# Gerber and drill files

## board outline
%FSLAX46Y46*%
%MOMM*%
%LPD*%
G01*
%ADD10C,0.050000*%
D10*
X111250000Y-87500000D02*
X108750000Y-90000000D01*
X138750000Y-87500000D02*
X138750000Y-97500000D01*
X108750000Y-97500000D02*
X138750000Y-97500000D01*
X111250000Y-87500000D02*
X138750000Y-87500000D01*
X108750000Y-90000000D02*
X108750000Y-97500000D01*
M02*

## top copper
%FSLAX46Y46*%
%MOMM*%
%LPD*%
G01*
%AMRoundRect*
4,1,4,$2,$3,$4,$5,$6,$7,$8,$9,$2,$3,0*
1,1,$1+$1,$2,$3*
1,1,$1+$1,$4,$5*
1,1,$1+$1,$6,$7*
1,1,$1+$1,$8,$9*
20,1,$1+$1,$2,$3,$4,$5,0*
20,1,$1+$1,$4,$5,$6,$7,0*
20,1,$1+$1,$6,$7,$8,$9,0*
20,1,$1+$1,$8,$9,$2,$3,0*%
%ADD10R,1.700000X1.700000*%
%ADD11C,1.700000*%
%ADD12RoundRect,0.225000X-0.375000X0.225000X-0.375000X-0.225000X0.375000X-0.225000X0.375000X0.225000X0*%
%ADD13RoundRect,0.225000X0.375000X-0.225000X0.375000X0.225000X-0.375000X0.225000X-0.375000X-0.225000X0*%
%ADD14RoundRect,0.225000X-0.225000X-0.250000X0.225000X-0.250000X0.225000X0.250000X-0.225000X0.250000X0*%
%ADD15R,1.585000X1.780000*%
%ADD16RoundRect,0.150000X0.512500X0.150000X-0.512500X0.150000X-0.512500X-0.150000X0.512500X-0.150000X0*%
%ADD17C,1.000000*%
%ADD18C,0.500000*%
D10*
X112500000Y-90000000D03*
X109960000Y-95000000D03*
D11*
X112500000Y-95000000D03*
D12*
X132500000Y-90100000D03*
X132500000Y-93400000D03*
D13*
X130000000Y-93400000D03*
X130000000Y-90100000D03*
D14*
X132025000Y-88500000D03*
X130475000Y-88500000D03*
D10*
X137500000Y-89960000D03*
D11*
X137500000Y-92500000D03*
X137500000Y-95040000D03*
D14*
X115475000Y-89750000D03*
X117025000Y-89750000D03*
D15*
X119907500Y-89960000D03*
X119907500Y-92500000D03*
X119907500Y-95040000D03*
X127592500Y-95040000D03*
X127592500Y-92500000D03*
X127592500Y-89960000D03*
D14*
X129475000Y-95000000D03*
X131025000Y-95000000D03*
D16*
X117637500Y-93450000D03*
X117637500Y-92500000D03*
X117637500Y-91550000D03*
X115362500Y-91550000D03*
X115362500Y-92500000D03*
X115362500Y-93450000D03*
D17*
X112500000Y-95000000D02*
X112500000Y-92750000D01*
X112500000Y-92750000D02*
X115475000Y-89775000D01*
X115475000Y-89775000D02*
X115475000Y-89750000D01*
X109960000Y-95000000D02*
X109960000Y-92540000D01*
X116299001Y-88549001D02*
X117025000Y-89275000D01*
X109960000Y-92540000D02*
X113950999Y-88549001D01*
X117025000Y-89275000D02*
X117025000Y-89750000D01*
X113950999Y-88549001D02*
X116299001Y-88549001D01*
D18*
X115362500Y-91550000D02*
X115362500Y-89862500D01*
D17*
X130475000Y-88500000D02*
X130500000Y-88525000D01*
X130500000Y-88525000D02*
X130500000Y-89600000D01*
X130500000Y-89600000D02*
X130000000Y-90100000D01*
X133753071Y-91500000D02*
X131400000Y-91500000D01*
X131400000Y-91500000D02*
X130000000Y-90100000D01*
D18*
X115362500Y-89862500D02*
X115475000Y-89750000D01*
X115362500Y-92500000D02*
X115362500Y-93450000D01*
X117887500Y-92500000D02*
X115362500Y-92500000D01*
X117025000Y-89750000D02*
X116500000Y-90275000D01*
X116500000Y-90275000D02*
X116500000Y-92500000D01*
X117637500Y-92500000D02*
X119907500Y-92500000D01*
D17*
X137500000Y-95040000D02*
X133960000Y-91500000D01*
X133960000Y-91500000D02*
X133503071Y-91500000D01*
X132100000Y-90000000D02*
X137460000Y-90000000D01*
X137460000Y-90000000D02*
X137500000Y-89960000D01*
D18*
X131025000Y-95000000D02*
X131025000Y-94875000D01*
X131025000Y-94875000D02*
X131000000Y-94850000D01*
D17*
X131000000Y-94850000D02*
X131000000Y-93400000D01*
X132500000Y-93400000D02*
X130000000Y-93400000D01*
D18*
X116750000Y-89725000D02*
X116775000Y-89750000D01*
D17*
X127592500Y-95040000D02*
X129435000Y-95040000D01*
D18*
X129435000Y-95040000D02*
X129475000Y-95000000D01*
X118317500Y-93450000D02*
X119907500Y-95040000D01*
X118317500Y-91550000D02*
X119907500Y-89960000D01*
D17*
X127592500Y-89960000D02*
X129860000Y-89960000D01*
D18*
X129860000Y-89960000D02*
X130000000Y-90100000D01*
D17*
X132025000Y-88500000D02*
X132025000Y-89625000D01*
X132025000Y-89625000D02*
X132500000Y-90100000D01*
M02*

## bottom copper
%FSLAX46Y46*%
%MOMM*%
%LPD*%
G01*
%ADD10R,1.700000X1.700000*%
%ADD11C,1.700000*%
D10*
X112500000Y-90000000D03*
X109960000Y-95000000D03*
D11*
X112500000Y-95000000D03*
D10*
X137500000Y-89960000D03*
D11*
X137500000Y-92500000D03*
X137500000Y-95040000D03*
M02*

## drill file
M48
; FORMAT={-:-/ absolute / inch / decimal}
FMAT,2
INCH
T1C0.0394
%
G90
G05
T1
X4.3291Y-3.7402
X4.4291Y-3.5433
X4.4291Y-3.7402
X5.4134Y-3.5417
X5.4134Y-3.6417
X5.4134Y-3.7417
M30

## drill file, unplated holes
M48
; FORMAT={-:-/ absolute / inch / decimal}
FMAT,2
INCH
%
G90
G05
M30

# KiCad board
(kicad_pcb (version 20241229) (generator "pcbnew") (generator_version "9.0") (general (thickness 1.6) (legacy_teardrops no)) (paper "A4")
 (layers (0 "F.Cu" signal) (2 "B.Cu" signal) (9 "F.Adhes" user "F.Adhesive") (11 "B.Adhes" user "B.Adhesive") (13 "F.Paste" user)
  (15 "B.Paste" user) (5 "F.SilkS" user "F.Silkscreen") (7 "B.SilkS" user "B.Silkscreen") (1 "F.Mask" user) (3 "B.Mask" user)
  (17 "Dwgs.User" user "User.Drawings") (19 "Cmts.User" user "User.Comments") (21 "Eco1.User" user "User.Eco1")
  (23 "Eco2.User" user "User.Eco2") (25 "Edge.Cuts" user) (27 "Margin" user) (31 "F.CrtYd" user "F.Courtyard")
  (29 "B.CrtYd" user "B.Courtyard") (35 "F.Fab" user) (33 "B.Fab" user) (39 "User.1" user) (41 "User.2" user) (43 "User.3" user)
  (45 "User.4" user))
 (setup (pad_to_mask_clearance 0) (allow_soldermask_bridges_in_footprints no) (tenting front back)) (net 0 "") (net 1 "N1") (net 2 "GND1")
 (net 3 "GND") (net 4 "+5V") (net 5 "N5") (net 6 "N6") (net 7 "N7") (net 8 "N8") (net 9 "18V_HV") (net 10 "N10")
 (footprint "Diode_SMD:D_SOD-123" (layer "F.Cu") (at 130 91.75 90)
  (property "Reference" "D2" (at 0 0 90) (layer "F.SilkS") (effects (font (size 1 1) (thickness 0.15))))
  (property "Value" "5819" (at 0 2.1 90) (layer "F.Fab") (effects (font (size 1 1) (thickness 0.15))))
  (pad "1" smd roundrect (at -1.65 0 90) (size 0.9 1.2) (layers "F.Cu" "F.Mask" "F.Paste") (roundrect_rratio 0.25) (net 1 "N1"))
  (pad "2" smd roundrect (at 1.65 0 90) (size 0.9 1.2) (layers "F.Cu" "F.Mask" "F.Paste") (roundrect_rratio 0.25) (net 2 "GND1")))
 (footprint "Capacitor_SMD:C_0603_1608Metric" (layer "F.Cu") (at 116.25 89.75)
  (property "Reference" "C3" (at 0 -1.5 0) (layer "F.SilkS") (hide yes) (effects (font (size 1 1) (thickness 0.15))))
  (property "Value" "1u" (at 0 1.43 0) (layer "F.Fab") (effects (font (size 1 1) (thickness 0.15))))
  (pad "1" smd roundrect (at -0.775 0) (size 0.9 0.95) (layers "F.Cu" "F.Mask" "F.Paste") (roundrect_rratio 0.25) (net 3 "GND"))
  (pad "2" smd roundrect (at 0.775 0) (size 0.9 0.95) (layers "F.Cu" "F.Mask" "F.Paste") (roundrect_rratio 0.25) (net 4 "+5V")))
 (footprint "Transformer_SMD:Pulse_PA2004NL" (layer "F.Cu") (at 123.75 92.5)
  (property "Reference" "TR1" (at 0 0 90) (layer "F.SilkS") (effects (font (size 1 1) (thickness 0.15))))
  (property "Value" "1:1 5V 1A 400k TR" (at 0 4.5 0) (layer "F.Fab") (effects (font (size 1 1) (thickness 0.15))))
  (pad "1" smd rect (at -3.8425 -2.54) (size 1.585 1.78) (layers "F.Cu" "F.Mask" "F.Paste") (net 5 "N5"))
  (pad "2" smd rect (at -3.8425 0) (size 1.585 1.78) (layers "F.Cu" "F.Mask" "F.Paste") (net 4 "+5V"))
  (pad "3" smd rect (at -3.8425 2.54) (size 1.585 1.78) (layers "F.Cu" "F.Mask" "F.Paste") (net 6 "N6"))
  (pad "4" smd rect (at 3.8425 2.54) (size 1.585 1.78) (layers "F.Cu" "F.Mask" "F.Paste") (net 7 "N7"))
  (pad "5" smd rect (at 3.8425 0) (size 1.585 1.78) (layers "F.Cu" "F.Mask" "F.Paste") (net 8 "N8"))
  (pad "6" smd rect (at 3.8425 -2.54) (size 1.585 1.78) (layers "F.Cu" "F.Mask" "F.Paste") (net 2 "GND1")))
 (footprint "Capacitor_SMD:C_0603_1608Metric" (layer "F.Cu") (at 130.25 95)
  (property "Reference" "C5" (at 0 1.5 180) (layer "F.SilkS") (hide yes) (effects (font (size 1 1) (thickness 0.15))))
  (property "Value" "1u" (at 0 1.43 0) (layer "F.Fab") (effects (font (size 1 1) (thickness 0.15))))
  (pad "1" smd roundrect (at -0.775 0) (size 0.9 0.95) (layers "F.Cu" "F.Mask" "F.Paste") (roundrect_rratio 0.25) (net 7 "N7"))
  (pad "2" smd roundrect (at 0.775 0) (size 0.9 0.95) (layers "F.Cu" "F.Mask" "F.Paste") (roundrect_rratio 0.25) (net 1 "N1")))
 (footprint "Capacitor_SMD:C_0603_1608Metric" (layer "F.Cu") (at 131.25 88.5)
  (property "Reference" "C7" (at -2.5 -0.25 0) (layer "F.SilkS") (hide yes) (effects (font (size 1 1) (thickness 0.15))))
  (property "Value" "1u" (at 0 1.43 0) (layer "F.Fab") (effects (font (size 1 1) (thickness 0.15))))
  (pad "1" smd roundrect (at -0.775 0) (size 0.9 0.95) (layers "F.Cu" "F.Mask" "F.Paste") (roundrect_rratio 0.25) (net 2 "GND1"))
  (pad "2" smd roundrect (at 0.775 0) (size 0.9 0.95) (layers "F.Cu" "F.Mask" "F.Paste") (roundrect_rratio 0.25) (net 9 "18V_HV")))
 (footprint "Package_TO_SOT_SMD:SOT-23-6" (layer "F.Cu") (at 116.5 92.5 180)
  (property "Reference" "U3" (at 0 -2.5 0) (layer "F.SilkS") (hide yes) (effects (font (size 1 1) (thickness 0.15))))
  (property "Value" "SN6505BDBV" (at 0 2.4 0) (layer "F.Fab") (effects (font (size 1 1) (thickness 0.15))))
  (pad "1" smd roundrect (at -1.1375 -0.95 180) (size 1.325 0.6) (layers "F.Cu" "F.Mask" "F.Paste") (roundrect_rratio 0.25) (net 6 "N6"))
  (pad "2" smd roundrect (at -1.1375 0 180) (size 1.325 0.6) (layers "F.Cu" "F.Mask" "F.Paste") (roundrect_rratio 0.25) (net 4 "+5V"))
  (pad "3" smd roundrect (at -1.1375 0.95 180) (size 1.325 0.6) (layers "F.Cu" "F.Mask" "F.Paste") (roundrect_rratio 0.25) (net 5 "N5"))
  (pad "4" smd roundrect (at 1.1375 0.95 180) (size 1.325 0.6) (layers "F.Cu" "F.Mask" "F.Paste") (roundrect_rratio 0.25) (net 3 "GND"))
  (pad "5" smd roundrect (at 1.1375 0 180) (size 1.325 0.6) (layers "F.Cu" "F.Mask" "F.Paste") (roundrect_rratio 0.25) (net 4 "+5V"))
  (pad "6" smd roundrect (at 1.1375 -0.95 180) (size 1.325 0.6) (layers "F.Cu" "F.Mask" "F.Paste") (roundrect_rratio 0.25) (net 4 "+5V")))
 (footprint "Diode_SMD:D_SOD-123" (layer "F.Cu") (at 132.5 91.75 -90)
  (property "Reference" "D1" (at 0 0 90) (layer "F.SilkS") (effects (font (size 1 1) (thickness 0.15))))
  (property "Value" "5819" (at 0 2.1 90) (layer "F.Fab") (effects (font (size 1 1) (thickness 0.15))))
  (pad "1" smd roundrect (at -1.65 0 270) (size 0.9 1.2) (layers "F.Cu" "F.Mask" "F.Paste") (roundrect_rratio 0.25) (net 9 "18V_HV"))
  (pad "2" smd roundrect (at 1.65 0 270) (size 0.9 1.2) (layers "F.Cu" "F.Mask" "F.Paste") (roundrect_rratio 0.25) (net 1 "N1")))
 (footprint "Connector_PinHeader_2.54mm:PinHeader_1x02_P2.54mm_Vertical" (layer "B.Cu") (at 109.96 95 -90)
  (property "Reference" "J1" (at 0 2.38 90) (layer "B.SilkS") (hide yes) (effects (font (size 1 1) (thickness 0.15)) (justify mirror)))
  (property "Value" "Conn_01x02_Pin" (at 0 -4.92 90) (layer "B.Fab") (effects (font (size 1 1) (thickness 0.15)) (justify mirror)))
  (pad "1" thru_hole rect (at 0 0 270) (size 1.7 1.7) (drill 1) (layers "*.Cu" "*.Mask") (remove_unused_layers no) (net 4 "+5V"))
  (pad "2" thru_hole circle (at 0 -2.54 270) (size 1.7 1.7) (drill 1) (layers "*.Cu" "*.Mask") (remove_unused_layers no) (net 3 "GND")))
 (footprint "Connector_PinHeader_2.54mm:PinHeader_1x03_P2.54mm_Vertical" (layer "B.Cu") (at 137.5 89.96 180)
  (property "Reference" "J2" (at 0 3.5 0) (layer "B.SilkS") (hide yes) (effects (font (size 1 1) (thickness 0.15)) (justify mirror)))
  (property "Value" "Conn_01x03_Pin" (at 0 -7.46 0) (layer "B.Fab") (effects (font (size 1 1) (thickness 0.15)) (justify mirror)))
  (pad "1" thru_hole rect (at 0 0 180) (size 1.7 1.7) (drill 1) (layers "*.Cu" "*.Mask") (remove_unused_layers no) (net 9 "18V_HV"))
  (pad "2" thru_hole circle (at 0 -2.54 180) (size 1.7 1.7) (drill 1) (layers "*.Cu" "*.Mask") (remove_unused_layers no) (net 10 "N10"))
  (pad "3" thru_hole circle (at 0 -5.08 180) (size 1.7 1.7) (drill 1) (layers "*.Cu" "*.Mask") (remove_unused_layers no) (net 2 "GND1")))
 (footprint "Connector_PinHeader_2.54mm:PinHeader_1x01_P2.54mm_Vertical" (layer "B.Cu") (at 112.5 90)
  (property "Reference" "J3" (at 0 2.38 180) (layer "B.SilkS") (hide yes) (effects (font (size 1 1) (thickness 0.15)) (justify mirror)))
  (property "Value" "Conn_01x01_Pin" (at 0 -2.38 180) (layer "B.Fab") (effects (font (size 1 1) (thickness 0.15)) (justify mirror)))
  (pad "1" thru_hole rect (at 0 0) (size 1.7 1.7) (drill 1) (layers "*.Cu" "*.Mask") (remove_unused_layers no) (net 4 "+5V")))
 (gr_line (start 111.25 87.5) (end 138.75 87.5) (stroke (width 0.05) (type default)) (layer "Edge.Cuts"))
 (gr_line (start 111.25 87.5) (end 108.75 90) (stroke (width 0.05) (type solid)) (layer "Edge.Cuts"))
 (gr_line (start 138.75 87.5) (end 138.75 97.5) (stroke (width 0.05) (type solid)) (layer "Edge.Cuts"))
 (gr_line (start 108.75 97.5) (end 138.75 97.5) (stroke (width 0.05) (type solid)) (layer "Edge.Cuts"))
 (gr_line (start 108.75 90) (end 108.75 97.5) (stroke (width 0.05) (type solid)) (layer "Edge.Cuts"))
 (segment (start 132.025 89.625) (end 132.5 90.1) (width 1) (layer "F.Cu") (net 9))
 (segment (start 132.1 90) (end 137.46 90) (width 1) (layer "F.Cu") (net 9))
 (segment (start 137.46 90) (end 137.5 89.96) (width 1) (layer "F.Cu") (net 9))
 (segment (start 132.025 88.5) (end 132.025 89.625) (width 1) (layer "F.Cu") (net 9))
 (segment (start 137.5 95.04) (end 133.96 91.5) (width 1) (layer "F.Cu") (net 2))
 (segment (start 130.5 88.525) (end 130.5 89.6) (width 1) (layer "F.Cu") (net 2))
 (segment (start 130.5 89.6) (end 130 90.1) (width 1) (layer "F.Cu") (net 2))
 (segment (start 131.4 91.5) (end 130 90.1) (width 1) (layer "F.Cu") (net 2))
 (segment (start 133.96 91.5) (end 133.503071 91.5) (width 1) (layer "F.Cu") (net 2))
 (segment (start 130.475 88.5) (end 130.5 88.525) (width 1) (layer "F.Cu") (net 2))
 (segment (start 133.753071 91.5) (end 131.4 91.5) (width 1) (layer "F.Cu") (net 2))
 (segment (start 129.86 89.96) (end 130 90.1) (width 0.5) (layer "F.Cu") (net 2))
 (segment (start 127.5925 89.96) (end 129.86 89.96) (width 1) (layer "F.Cu") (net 2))
 (segment (start 112.5 95) (end 112.5 92.75) (width 1) (layer "F.Cu") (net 3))
 (segment (start 115.3625 89.8625) (end 115.475 89.75) (width 0.5) (layer "F.Cu") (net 3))
 (segment (start 115.475 89.775) (end 115.475 89.75) (width 1) (layer "F.Cu") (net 3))
 (segment (start 112.5 92.75) (end 115.475 89.775) (width 1) (layer "F.Cu") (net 3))
 (segment (start 115.3625 91.55) (end 115.3625 89.8625) (width 0.5) (layer "F.Cu") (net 3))
 (segment (start 116.75 89.725) (end 116.775 89.75) (width 0.5) (layer "F.Cu") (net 4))
 (segment (start 117.025 89.275) (end 117.025 89.75) (width 1) (layer "F.Cu") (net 4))
 (segment (start 116.299001 88.549001) (end 117.025 89.275) (width 1) (layer "F.Cu") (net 4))
 (segment (start 116.5 90.275) (end 116.5 92.5) (width 0.5) (layer "F.Cu") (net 4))
 (segment (start 115.3625 92.5) (end 115.3625 93.45) (width 0.5) (layer "F.Cu") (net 4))
 (segment (start 109.96 95) (end 109.96 92.54) (width 1) (layer "F.Cu") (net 4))
 (segment (start 113.950999 88.549001) (end 116.299001 88.549001) (width 1) (layer "F.Cu") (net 4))
 (segment (start 117.8875 92.5) (end 115.3625 92.5) (width 0.5) (layer "F.Cu") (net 4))
 (segment (start 117.025 89.75) (end 116.5 90.275) (width 0.5) (layer "F.Cu") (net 4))
 (segment (start 117.6375 92.5) (end 119.9075 92.5) (width 0.5) (layer "F.Cu") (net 4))
 (segment (start 109.96 92.54) (end 113.950999 88.549001) (width 1) (layer "F.Cu") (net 4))
 (segment (start 127.5925 95.04) (end 129.435 95.04) (width 1) (layer "F.Cu") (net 7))
 (segment (start 129.435 95.04) (end 129.475 95) (width 0.5) (layer "F.Cu") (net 7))
 (segment (start 118.3175 93.45) (end 119.9075 95.04) (width 0.5) (layer "F.Cu") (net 6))
 (segment (start 118.3175 91.55) (end 119.9075 89.96) (width 0.5) (layer "F.Cu") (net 5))
 (segment (start 131.025 94.875) (end 131 94.85) (width 0.5) (layer "F.Cu") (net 1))
 (segment (start 131 94.85) (end 131 93.4) (width 1) (layer "F.Cu") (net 1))
 (segment (start 132.5 93.4) (end 130 93.4) (width 1) (layer "F.Cu") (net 1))
 (segment (start 131.025 95) (end 131.025 94.875) (width 0.5) (layer "F.Cu") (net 1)))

